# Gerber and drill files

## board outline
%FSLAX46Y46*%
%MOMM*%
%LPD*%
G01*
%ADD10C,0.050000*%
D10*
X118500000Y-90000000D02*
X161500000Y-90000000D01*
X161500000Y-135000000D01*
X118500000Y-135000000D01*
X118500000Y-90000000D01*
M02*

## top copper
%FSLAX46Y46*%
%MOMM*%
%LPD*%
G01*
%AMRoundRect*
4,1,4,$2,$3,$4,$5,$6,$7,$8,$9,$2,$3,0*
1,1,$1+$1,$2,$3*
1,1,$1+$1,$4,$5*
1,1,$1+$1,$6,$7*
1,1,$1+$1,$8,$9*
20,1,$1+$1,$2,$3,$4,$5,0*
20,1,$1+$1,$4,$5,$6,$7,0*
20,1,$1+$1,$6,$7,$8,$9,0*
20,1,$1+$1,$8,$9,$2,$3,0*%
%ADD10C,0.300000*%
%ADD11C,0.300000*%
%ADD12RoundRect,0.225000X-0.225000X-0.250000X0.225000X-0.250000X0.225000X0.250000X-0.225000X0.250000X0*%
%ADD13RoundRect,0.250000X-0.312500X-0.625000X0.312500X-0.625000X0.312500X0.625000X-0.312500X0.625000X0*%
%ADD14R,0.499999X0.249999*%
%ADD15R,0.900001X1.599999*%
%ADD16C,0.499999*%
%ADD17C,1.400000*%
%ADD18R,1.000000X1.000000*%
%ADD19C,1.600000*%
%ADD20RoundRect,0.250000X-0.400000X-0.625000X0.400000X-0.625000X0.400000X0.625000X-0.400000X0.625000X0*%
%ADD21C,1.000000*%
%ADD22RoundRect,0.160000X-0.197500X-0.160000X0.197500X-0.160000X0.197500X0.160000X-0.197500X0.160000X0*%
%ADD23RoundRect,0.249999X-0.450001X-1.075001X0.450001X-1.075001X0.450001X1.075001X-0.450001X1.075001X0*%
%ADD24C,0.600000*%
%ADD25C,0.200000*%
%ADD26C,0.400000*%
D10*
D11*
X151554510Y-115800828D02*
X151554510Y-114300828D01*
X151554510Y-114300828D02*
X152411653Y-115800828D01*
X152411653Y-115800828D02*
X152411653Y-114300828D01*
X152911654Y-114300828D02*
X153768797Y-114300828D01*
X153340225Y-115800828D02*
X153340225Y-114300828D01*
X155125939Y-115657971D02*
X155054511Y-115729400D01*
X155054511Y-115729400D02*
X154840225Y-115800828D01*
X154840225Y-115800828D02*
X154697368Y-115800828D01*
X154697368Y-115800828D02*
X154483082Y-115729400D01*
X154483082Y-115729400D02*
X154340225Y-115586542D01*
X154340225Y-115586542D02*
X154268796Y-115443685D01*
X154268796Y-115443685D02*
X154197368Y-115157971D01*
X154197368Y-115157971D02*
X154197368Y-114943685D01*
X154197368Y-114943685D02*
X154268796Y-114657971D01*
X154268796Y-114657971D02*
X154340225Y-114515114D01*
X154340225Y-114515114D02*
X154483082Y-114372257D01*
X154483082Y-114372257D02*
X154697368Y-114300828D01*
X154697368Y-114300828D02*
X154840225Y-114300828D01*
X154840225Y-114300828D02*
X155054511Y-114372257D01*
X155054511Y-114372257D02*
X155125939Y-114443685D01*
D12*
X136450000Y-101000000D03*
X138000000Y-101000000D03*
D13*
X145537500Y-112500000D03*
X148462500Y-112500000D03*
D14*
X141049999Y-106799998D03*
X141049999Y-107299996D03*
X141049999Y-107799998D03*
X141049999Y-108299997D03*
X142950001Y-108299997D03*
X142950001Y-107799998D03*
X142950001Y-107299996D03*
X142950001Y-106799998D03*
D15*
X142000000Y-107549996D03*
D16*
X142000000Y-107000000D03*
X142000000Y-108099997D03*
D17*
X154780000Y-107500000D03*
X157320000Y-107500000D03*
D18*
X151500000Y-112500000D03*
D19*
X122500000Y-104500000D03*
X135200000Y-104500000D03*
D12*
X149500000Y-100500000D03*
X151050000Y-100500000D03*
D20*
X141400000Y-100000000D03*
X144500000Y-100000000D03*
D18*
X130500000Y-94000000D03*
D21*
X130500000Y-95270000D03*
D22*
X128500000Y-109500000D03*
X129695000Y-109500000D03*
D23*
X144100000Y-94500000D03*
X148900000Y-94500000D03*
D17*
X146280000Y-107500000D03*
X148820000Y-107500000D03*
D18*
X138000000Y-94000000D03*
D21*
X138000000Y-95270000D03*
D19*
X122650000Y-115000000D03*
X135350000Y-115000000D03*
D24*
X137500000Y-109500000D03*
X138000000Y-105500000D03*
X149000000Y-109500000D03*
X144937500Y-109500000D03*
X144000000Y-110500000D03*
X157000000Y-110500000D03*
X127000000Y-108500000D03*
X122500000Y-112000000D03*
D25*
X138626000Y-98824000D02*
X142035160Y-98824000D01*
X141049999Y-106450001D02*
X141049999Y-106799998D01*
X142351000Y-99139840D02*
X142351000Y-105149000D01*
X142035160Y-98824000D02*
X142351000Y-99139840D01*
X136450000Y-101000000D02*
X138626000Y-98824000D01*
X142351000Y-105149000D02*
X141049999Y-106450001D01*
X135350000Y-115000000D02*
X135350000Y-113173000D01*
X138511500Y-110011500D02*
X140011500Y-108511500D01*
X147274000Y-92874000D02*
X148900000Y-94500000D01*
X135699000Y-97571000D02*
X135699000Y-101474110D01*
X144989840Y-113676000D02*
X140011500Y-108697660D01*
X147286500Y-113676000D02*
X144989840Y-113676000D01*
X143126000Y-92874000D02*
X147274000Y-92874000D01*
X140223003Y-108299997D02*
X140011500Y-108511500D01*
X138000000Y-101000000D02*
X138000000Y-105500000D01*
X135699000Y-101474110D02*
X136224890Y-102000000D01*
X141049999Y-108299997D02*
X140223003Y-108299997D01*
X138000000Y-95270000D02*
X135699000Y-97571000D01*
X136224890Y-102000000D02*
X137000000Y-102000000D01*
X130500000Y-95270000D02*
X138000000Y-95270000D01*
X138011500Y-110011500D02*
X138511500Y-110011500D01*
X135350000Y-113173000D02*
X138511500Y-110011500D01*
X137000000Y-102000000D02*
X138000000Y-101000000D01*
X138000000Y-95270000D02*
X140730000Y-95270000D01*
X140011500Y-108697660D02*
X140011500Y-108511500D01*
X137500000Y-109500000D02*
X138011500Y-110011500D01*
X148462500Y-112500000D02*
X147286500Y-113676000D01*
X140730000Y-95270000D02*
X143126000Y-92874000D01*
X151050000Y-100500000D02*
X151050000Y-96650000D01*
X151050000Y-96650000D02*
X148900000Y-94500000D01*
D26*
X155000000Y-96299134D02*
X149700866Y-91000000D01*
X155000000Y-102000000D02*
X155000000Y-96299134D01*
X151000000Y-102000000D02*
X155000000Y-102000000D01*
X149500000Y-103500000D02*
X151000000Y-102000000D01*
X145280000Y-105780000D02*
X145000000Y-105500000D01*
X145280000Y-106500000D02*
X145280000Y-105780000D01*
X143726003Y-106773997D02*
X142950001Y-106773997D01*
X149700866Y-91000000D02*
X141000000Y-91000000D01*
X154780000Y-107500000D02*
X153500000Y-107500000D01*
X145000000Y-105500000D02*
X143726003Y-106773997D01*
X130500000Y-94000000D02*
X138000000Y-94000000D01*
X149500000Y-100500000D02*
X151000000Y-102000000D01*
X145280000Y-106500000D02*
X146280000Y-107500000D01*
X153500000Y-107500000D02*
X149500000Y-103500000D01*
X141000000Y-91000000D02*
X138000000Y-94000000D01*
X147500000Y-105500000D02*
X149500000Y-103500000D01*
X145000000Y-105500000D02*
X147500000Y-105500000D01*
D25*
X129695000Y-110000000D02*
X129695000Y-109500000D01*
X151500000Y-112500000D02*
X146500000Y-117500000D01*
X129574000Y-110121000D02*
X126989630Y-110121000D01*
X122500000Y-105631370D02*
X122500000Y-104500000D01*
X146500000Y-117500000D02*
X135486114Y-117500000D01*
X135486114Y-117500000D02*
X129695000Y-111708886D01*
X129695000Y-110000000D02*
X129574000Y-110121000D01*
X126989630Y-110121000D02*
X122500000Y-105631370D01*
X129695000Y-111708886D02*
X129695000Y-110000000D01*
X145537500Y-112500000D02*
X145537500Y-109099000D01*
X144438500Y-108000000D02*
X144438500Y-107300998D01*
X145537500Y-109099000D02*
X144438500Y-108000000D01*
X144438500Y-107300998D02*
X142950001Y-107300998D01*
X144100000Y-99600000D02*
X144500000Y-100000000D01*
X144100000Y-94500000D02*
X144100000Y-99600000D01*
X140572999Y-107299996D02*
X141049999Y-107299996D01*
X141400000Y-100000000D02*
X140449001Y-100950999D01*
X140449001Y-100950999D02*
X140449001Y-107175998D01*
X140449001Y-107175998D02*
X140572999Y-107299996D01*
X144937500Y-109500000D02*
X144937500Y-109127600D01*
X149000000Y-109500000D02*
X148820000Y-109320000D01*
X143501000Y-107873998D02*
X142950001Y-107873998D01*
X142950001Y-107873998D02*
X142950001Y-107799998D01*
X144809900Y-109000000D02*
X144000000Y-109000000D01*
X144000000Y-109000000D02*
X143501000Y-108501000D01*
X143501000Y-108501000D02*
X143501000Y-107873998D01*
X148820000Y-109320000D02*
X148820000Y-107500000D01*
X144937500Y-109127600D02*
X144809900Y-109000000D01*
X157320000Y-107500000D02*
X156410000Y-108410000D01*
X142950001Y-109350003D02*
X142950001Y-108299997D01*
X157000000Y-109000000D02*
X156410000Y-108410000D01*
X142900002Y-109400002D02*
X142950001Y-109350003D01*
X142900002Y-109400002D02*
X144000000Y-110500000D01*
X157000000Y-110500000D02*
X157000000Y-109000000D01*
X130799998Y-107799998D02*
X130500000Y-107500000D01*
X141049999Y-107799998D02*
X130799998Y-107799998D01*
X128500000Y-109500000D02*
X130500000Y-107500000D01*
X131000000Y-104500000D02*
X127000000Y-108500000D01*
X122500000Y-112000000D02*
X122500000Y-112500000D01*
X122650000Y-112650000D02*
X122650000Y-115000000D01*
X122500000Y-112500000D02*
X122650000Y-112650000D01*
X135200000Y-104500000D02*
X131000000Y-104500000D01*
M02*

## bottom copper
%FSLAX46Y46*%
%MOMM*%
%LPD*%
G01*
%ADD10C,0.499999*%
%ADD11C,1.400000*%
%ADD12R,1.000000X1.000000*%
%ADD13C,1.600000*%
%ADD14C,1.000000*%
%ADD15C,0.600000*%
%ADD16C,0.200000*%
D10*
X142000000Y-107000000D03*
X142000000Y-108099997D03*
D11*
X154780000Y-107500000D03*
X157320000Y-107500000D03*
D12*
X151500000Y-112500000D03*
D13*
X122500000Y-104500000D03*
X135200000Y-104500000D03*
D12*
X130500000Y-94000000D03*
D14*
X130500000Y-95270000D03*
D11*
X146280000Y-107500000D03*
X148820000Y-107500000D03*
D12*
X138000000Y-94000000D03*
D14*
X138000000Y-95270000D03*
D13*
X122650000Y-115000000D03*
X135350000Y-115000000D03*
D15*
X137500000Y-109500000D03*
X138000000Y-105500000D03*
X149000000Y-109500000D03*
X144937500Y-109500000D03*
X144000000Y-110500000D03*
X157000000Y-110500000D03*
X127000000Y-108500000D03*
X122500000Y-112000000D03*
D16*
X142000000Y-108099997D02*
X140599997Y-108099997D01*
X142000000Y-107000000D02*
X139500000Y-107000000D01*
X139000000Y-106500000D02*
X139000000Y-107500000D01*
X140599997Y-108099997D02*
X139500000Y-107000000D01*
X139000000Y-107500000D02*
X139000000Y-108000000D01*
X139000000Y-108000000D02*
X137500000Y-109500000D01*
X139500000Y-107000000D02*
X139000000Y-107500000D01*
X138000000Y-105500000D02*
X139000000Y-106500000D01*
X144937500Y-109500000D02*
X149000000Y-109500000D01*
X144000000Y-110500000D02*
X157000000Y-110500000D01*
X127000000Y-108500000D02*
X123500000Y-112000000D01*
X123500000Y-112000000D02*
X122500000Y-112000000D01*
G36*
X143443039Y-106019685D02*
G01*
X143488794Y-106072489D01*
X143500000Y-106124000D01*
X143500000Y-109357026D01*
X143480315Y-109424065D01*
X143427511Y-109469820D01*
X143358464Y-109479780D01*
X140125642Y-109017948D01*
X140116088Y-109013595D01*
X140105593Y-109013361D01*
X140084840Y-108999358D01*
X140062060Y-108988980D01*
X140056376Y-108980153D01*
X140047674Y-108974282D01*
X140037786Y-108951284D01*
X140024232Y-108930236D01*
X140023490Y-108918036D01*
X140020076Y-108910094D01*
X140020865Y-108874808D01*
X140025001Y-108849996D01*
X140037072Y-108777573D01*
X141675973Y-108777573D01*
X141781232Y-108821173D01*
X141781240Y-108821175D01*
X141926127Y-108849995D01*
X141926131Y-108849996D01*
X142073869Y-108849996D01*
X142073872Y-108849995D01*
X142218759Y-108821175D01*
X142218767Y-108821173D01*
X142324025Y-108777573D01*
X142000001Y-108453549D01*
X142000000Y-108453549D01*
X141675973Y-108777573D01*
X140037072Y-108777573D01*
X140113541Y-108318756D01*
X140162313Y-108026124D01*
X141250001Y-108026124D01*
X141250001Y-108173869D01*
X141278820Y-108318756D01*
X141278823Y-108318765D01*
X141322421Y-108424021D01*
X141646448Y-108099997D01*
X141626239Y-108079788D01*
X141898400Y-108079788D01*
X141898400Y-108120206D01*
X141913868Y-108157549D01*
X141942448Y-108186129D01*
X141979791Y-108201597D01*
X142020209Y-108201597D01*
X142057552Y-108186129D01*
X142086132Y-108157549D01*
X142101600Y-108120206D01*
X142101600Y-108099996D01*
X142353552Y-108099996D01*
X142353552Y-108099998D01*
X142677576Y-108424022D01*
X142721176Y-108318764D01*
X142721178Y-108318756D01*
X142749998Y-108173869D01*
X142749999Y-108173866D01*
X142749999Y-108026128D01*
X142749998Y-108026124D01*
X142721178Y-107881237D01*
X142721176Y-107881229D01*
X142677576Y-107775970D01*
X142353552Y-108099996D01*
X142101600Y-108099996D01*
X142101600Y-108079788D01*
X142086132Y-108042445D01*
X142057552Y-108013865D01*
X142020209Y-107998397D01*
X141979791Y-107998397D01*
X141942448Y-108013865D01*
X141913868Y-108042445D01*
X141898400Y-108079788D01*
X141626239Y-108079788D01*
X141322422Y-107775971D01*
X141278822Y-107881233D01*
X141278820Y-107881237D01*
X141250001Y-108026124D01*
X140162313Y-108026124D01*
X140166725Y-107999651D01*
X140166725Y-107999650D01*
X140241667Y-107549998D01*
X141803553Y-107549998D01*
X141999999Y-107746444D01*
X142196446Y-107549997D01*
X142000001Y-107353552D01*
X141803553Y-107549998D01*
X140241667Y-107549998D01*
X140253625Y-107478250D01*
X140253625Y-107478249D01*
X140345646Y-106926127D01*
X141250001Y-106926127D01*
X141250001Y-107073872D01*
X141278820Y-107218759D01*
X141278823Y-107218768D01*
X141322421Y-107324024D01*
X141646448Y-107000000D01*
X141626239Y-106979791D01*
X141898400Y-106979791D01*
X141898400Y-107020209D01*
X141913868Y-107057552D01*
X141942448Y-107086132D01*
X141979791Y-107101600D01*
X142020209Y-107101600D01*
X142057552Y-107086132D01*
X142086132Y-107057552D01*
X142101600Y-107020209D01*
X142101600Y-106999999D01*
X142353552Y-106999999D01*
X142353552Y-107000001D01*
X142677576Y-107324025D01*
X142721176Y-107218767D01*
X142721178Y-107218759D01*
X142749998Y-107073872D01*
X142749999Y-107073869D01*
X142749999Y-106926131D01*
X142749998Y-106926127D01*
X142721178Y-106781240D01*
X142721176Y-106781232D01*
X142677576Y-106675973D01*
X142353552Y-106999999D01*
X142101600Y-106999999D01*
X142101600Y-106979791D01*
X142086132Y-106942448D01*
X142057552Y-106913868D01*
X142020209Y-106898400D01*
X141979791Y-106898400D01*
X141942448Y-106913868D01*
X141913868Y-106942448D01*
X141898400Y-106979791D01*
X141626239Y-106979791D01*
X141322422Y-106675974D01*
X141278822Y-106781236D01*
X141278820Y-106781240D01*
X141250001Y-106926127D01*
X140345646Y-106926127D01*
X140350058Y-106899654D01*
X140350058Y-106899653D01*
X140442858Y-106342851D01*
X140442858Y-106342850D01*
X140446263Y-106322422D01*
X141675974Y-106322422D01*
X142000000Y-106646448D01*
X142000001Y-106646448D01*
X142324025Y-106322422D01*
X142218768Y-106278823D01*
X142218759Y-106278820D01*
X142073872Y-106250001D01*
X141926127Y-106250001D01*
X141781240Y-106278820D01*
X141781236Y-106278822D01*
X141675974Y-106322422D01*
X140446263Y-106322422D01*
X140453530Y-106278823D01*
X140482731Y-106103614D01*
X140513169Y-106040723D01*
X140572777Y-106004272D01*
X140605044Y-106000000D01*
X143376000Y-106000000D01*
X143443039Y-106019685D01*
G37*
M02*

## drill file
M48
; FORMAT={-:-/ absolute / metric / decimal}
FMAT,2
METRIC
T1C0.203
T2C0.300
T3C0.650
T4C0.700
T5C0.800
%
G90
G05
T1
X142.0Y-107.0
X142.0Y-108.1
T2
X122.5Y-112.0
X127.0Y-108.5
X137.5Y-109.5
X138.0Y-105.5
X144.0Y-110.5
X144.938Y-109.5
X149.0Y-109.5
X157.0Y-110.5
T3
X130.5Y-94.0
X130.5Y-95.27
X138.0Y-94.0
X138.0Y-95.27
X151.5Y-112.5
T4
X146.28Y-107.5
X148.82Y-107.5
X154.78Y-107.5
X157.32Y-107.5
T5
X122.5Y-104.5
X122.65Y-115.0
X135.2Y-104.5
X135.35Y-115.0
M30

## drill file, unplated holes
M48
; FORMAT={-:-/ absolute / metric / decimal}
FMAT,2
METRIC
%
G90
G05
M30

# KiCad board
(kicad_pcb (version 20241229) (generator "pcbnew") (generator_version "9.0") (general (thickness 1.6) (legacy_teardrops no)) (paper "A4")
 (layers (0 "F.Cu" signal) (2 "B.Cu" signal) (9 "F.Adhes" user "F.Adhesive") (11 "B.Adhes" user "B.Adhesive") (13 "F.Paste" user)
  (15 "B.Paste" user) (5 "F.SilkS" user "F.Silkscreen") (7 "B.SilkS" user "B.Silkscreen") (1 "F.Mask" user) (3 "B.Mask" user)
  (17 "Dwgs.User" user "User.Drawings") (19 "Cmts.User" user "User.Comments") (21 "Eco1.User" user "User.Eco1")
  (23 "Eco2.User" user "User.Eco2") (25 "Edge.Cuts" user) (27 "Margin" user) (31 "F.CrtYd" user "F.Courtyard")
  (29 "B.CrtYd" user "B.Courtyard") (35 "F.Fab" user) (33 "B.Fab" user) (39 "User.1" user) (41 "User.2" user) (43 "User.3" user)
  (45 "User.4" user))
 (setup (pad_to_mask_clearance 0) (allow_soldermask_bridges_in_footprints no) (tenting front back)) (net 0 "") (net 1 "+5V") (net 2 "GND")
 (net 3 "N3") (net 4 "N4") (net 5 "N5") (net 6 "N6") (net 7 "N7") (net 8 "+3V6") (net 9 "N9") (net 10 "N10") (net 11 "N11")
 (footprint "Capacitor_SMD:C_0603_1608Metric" (layer "F.Cu") (at 137.225 101)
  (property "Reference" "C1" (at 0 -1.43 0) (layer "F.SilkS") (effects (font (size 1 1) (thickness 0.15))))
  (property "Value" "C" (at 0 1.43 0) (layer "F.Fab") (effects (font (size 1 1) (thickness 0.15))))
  (pad "1" smd roundrect (at -0.775 0) (size 0.9 0.95) (layers "F.Cu" "F.Mask" "F.Paste") (roundrect_rratio 0.25) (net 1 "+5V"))
  (pad "2" smd roundrect (at 0.775 0) (size 0.9 0.95) (layers "F.Cu" "F.Mask" "F.Paste") (roundrect_rratio 0.25) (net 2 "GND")))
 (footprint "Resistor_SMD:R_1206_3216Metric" (layer "F.Cu") (at 147 112.5)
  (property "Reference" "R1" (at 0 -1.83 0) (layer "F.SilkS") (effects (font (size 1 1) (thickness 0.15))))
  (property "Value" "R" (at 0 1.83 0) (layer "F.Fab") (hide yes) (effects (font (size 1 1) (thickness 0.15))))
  (pad "1" smd roundrect (at -1.4625 0) (size 1.125 1.75) (layers "F.Cu" "F.Mask" "F.Paste") (roundrect_rratio 0.222222) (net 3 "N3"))
  (pad "2" smd roundrect (at 1.4625 0) (size 1.125 1.75) (layers "F.Cu" "F.Mask" "F.Paste") (roundrect_rratio 0.222222) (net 2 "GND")))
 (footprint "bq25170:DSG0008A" (layer "F.Cu") (at 142 107.549996)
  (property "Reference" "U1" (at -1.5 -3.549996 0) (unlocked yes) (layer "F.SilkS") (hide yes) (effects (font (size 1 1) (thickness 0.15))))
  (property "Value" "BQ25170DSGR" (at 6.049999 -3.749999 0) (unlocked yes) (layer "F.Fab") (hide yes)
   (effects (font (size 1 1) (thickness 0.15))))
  (pad "1" smd rect (at -0.950001 -0.749998 90) (size 0.249999 0.499999) (layers "F.Cu" "F.Mask" "F.Paste") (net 1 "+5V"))
  (pad "2" smd rect (at -0.950001 -0.25 90) (size 0.249999 0.499999) (layers "F.Cu" "F.Mask" "F.Paste") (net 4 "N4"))
  (pad "3" smd rect (at -0.950001 0.250002 90) (size 0.249999 0.499999) (layers "F.Cu" "F.Mask" "F.Paste") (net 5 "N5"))
  (pad "4" smd rect (at -0.950001 0.750001 90) (size 0.249999 0.499999) (layers "F.Cu" "F.Mask" "F.Paste") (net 2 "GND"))
  (pad "5" smd rect (at 0.950001 0.750001 90) (size 0.249999 0.499999) (layers "F.Cu" "F.Mask" "F.Paste") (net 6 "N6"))
  (pad "6" smd rect (at 0.950001 0.250002 90) (size 0.249999 0.499999) (layers "F.Cu" "F.Mask" "F.Paste") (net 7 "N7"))
  (pad "7" smd rect (at 0.950001 -0.25 90) (size 0.249999 0.499999) (layers "F.Cu" "F.Mask" "F.Paste") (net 3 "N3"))
  (pad "8" smd rect (at 0.950001 -0.749998 90) (size 0.249999 0.499999) (layers "F.Cu" "F.Mask" "F.Paste") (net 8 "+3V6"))
  (pad "9" smd rect (at 0 0) (size 0.900001 1.599999) (layers "F.Cu" "F.Mask" "F.Paste") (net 2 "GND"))
  (pad "10" thru_hole circle (at 0 -0.549996) (size 0.499999 0.499999) (drill 0.2032) (layers "*.Cu" "*.Mask") (remove_unused_layers yes)
   (keep_end_layers yes) (zone_layer_connections) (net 2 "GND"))
  (pad "11" thru_hole circle (at 0 0.550001) (size 0.499999 0.499999) (drill 0.2032) (layers "*.Cu" "*.Mask") (remove_unused_layers yes)
   (keep_end_layers yes) (zone_layer_connections) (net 2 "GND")))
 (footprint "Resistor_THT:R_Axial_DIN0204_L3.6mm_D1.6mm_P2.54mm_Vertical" (layer "F.Cu") (at 154.78 107.5)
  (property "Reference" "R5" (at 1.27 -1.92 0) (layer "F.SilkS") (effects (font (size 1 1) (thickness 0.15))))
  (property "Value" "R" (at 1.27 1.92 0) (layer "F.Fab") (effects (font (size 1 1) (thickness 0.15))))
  (pad "1" thru_hole circle (at 0 0) (size 1.4 1.4) (drill 0.7) (layers "*.Cu" "*.Mask") (remove_unused_layers yes) (keep_end_layers yes)
   (zone_layer_connections) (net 8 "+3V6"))
  (pad "2" thru_hole circle (at 2.54 0) (size 1.4 1.4) (drill 0.7) (layers "*.Cu" "*.Mask") (remove_unused_layers yes) (keep_end_layers yes)
   (zone_layer_connections) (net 6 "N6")))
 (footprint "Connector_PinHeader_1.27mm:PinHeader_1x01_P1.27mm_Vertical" (layer "F.Cu") (at 151.5 112.5)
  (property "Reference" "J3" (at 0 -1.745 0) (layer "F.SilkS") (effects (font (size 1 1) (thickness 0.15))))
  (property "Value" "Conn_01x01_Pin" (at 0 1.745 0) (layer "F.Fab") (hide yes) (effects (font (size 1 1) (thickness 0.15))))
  (pad "1" thru_hole rect (at 0 0) (size 1 1) (drill 0.65) (layers "*.Cu" "*.Mask") (remove_unused_layers yes) (keep_end_layers yes)
   (zone_layer_connections) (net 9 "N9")))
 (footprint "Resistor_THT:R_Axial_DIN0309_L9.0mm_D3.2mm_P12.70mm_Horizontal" (layer "F.Cu") (at 122.5 104.5)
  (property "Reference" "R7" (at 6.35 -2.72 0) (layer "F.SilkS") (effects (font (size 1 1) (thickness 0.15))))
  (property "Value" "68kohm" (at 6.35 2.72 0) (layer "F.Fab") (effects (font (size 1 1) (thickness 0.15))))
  (pad "1" thru_hole circle (at 0 0) (size 1.6 1.6) (drill 0.8) (layers "*.Cu" "*.Mask") (remove_unused_layers yes) (keep_end_layers yes)
   (zone_layer_connections) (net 9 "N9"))
  (pad "2" thru_hole circle (at 12.7 0) (size 1.6 1.6) (drill 0.8) (layers "*.Cu" "*.Mask") (remove_unused_layers yes) (keep_end_layers yes)
   (zone_layer_connections) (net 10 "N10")))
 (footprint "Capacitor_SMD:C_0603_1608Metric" (layer "F.Cu") (at 150.275 100.5)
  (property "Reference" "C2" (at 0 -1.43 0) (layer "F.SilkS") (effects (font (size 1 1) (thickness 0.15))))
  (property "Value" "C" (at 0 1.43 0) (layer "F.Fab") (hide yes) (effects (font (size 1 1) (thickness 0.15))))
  (pad "1" smd roundrect (at -0.775 0) (size 0.9 0.95) (layers "F.Cu" "F.Mask" "F.Paste") (roundrect_rratio 0.25) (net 8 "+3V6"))
  (pad "2" smd roundrect (at 0.775 0) (size 0.9 0.95) (layers "F.Cu" "F.Mask" "F.Paste") (roundrect_rratio 0.25) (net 2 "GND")))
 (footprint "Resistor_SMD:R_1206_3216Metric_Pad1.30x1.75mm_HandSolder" (layer "F.Cu") (at 142.95 100)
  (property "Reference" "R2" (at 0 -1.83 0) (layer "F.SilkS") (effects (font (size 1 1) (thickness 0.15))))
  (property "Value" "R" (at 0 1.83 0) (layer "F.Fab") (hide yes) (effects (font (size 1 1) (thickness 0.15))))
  (pad "1" smd roundrect (at -1.55 0) (size 1.3 1.75) (layers "F.Cu" "F.Mask" "F.Paste") (roundrect_rratio 0.192308) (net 4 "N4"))
  (pad "2" smd roundrect (at 1.55 0) (size 1.3 1.75) (layers "F.Cu" "F.Mask" "F.Paste") (roundrect_rratio 0.192308) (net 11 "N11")))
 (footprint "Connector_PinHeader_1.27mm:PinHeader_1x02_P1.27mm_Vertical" (layer "F.Cu") (at 130.5 94)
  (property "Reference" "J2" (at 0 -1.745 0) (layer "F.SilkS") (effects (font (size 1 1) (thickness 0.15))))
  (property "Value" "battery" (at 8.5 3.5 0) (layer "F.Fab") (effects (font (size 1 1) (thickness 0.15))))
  (pad "1" thru_hole rect (at 0 0) (size 1 1) (drill 0.65) (layers "*.Cu" "*.Mask") (remove_unused_layers yes) (keep_end_layers yes)
   (zone_layer_connections) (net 8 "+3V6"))
  (pad "2" thru_hole circle (at 0 1.27) (size 1 1) (drill 0.65) (layers "*.Cu" "*.Mask") (remove_unused_layers yes) (keep_end_layers yes)
   (zone_layer_connections) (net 2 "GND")))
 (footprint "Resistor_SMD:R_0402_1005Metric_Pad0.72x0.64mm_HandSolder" (layer "F.Cu") (at 129.0975 109.5)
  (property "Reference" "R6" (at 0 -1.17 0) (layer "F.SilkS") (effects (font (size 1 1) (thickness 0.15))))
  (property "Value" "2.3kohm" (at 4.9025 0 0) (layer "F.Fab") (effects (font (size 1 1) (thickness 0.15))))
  (pad "1" smd roundrect (at -0.5975 0) (size 0.715 0.64) (layers "F.Cu" "F.Mask" "F.Paste") (roundrect_rratio 0.25) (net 5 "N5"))
  (pad "2" smd roundrect (at 0.5975 0) (size 0.715 0.64) (layers "F.Cu" "F.Mask" "F.Paste") (roundrect_rratio 0.25) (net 9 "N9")))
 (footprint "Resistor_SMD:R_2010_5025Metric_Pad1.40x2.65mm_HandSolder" (layer "F.Cu") (at 146.5 94.5)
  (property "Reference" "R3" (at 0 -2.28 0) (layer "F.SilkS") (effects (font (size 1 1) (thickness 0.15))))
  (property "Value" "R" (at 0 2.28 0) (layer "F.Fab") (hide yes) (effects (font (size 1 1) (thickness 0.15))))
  (pad "1" smd roundrect (at -2.4 0) (size 1.4 2.65) (layers "F.Cu" "F.Mask" "F.Paste") (roundrect_rratio 0.178571) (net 11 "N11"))
  (pad "2" smd roundrect (at 2.4 0) (size 1.4 2.65) (layers "F.Cu" "F.Mask" "F.Paste") (roundrect_rratio 0.178571) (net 2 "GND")))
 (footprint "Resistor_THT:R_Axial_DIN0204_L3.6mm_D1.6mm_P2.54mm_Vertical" (layer "F.Cu") (at 146.28 107.5)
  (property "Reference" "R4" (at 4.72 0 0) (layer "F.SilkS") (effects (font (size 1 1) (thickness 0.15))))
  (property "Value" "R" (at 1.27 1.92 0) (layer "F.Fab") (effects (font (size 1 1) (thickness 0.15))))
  (pad "1" thru_hole circle (at 0 0) (size 1.4 1.4) (drill 0.7) (layers "*.Cu" "*.Mask") (remove_unused_layers yes) (keep_end_layers yes)
   (zone_layer_connections) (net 8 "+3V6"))
  (pad "2" thru_hole circle (at 2.54 0) (size 1.4 1.4) (drill 0.7) (layers "*.Cu" "*.Mask") (remove_unused_layers yes) (keep_end_layers yes)
   (zone_layer_connections) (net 7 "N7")))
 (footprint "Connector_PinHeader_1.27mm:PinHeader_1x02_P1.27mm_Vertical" (layer "F.Cu") (at 138 94)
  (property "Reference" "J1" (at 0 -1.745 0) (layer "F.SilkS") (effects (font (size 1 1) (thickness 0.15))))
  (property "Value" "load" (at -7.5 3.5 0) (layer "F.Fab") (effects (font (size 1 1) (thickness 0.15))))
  (pad "1" thru_hole rect (at 0 0) (size 1 1) (drill 0.65) (layers "*.Cu" "*.Mask") (remove_unused_layers yes) (keep_end_layers yes)
   (zone_layer_connections) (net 8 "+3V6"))
  (pad "2" thru_hole circle (at 0 1.27) (size 1 1) (drill 0.65) (layers "*.Cu" "*.Mask") (remove_unused_layers yes) (keep_end_layers yes)
   (zone_layer_connections) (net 2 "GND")))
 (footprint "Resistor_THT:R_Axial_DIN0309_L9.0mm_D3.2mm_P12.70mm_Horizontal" (layer "F.Cu") (at 122.65 115)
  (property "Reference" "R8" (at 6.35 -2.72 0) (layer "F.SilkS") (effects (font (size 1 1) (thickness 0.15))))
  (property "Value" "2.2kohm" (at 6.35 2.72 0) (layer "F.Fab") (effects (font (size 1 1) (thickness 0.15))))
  (pad "1" thru_hole circle (at 0 0) (size 1.6 1.6) (drill 0.8) (layers "*.Cu" "*.Mask") (remove_unused_layers yes) (keep_end_layers yes)
   (zone_layer_connections) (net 10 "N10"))
  (pad "2" thru_hole circle (at 12.7 0) (size 1.6 1.6) (drill 0.8) (layers "*.Cu" "*.Mask") (remove_unused_layers yes) (keep_end_layers yes)
   (zone_layer_connections) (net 2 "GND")))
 (gr_rect (start 118.5 90) (end 161.5 135) (stroke (width 0.05) (type default)) (fill no) (layer "Edge.Cuts"))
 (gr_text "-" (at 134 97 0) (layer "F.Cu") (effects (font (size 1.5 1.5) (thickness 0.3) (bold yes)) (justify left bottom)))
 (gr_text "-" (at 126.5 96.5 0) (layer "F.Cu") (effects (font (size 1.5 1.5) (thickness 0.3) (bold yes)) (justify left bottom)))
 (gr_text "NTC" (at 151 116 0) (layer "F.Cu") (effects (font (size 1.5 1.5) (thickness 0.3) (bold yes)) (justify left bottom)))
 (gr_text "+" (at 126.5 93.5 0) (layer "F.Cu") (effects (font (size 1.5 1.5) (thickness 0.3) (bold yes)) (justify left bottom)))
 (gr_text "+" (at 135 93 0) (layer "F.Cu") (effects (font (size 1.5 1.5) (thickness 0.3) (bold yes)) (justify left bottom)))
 (segment (start 138.626 98.824) (end 142.03516 98.824) (width 0.2) (layer "F.Cu") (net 1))
 (segment (start 141.049999 106.450001) (end 141.049999 106.799998) (width 0.2) (layer "F.Cu") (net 1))
 (segment (start 142.351 99.13984) (end 142.351 105.149) (width 0.2) (layer "F.Cu") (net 1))
 (segment (start 142.03516 98.824) (end 142.351 99.13984) (width 0.2) (layer "F.Cu") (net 1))
 (segment (start 136.45 101) (end 138.626 98.824) (width 0.2) (layer "F.Cu") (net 1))
 (segment (start 142.351 105.149) (end 141.049999 106.450001) (width 0.2) (layer "F.Cu") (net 1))
 (segment (start 135.35 115) (end 135.35 113.173) (width 0.2) (layer "F.Cu") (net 2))
 (segment (start 138.5115 110.0115) (end 140.0115 108.5115) (width 0.2) (layer "F.Cu") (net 2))
 (segment (start 147.274 92.874) (end 148.9 94.5) (width 0.2) (layer "F.Cu") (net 2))
 (segment (start 135.699 97.571) (end 135.699 101.47411) (width 0.2) (layer "F.Cu") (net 2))
 (segment (start 144.98984 113.676) (end 140.0115 108.69766) (width 0.2) (layer "F.Cu") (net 2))
 (segment (start 147.2865 113.676) (end 144.98984 113.676) (width 0.2) (layer "F.Cu") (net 2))
 (segment (start 143.126 92.874) (end 147.274 92.874) (width 0.2) (layer "F.Cu") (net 2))
 (segment (start 140.223003 108.299997) (end 140.0115 108.5115) (width 0.2) (layer "F.Cu") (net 2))
 (segment (start 138 101) (end 138 105.5) (width 0.2) (layer "F.Cu") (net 2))
 (segment (start 135.699 101.47411) (end 136.22489 102) (width 0.2) (layer "F.Cu") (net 2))
 (segment (start 141.049999 108.299997) (end 140.223003 108.299997) (width 0.2) (layer "F.Cu") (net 2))
 (segment (start 138 95.27) (end 135.699 97.571) (width 0.2) (layer "F.Cu") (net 2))
 (segment (start 136.22489 102) (end 137 102) (width 0.2) (layer "F.Cu") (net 2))
 (segment (start 130.5 95.27) (end 138 95.27) (width 0.2) (layer "F.Cu") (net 2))
 (segment (start 138.0115 110.0115) (end 138.5115 110.0115) (width 0.2) (layer "F.Cu") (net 2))
 (segment (start 135.35 113.173) (end 138.5115 110.0115) (width 0.2) (layer "F.Cu") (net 2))
 (segment (start 137 102) (end 138 101) (width 0.2) (layer "F.Cu") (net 2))
 (segment (start 138 95.27) (end 140.73 95.27) (width 0.2) (layer "F.Cu") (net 2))
 (segment (start 140.0115 108.69766) (end 140.0115 108.5115) (width 0.2) (layer "F.Cu") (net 2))
 (segment (start 137.5 109.5) (end 138.0115 110.0115) (width 0.2) (layer "F.Cu") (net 2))
 (segment (start 148.4625 112.5) (end 147.2865 113.676) (width 0.2) (layer "F.Cu") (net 2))
 (segment (start 140.73 95.27) (end 143.126 92.874) (width 0.2) (layer "F.Cu") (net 2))
 (segment (start 151.05 100.5) (end 151.05 96.65) (width 0.2) (layer "F.Cu") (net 2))
 (segment (start 151.05 96.65) (end 148.9 94.5) (width 0.2) (layer "F.Cu") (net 2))
 (via (at 137.5 109.5) (size 0.6) (drill 0.3) (layers "F.Cu" "B.Cu") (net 2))
 (via (at 138 105.5) (size 0.6) (drill 0.3) (layers "F.Cu" "B.Cu") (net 2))
 (segment (start 142 108.099997) (end 140.599997 108.099997) (width 0.2) (layer "B.Cu") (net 2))
 (segment (start 142 107) (end 139.5 107) (width 0.2) (layer "B.Cu") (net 2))
 (segment (start 139 106.5) (end 139 107.5) (width 0.2) (layer "B.Cu") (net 2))
 (segment (start 140.599997 108.099997) (end 139.5 107) (width 0.2) (layer "B.Cu") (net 2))
 (segment (start 139 107.5) (end 139 108) (width 0.2) (layer "B.Cu") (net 2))
 (segment (start 139 108) (end 137.5 109.5) (width 0.2) (layer "B.Cu") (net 2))
 (segment (start 139.5 107) (end 139 107.5) (width 0.2) (layer "B.Cu") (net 2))
 (segment (start 138 105.5) (end 139 106.5) (width 0.2) (layer "B.Cu") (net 2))
 (segment (start 155 96.299134) (end 149.700866 91) (width 0.4) (layer "F.Cu") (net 8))
 (segment (start 155 102) (end 155 96.299134) (width 0.4) (layer "F.Cu") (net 8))
 (segment (start 151 102) (end 155 102) (width 0.4) (layer "F.Cu") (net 8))
 (segment (start 149.5 103.5) (end 151 102) (width 0.4) (layer "F.Cu") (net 8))
 (segment (start 145.28 105.78) (end 145 105.5) (width 0.4) (layer "F.Cu") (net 8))
 (segment (start 145.28 106.5) (end 145.28 105.78) (width 0.4) (layer "F.Cu") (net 8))
 (segment (start 143.726003 106.773997) (end 142.950001 106.773997) (width 0.4) (layer "F.Cu") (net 8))
 (segment (start 149.700866 91) (end 141 91) (width 0.4) (layer "F.Cu") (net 8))
 (segment (start 154.78 107.5) (end 153.5 107.5) (width 0.4) (layer "F.Cu") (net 8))
 (segment (start 145 105.5) (end 143.726003 106.773997) (width 0.4) (layer "F.Cu") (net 8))
 (segment (start 130.5 94) (end 138 94) (width 0.4) (layer "F.Cu") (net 8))
 (segment (start 149.5 100.5) (end 151 102) (width 0.4) (layer "F.Cu") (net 8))
 (segment (start 145.28 106.5) (end 146.28 107.5) (width 0.4) (layer "F.Cu") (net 8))
 (segment (start 153.5 107.5) (end 149.5 103.5) (width 0.4) (layer "F.Cu") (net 8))
 (segment (start 141 91) (end 138 94) (width 0.4) (layer "F.Cu") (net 8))
 (segment (start 147.5 105.5) (end 149.5 103.5) (width 0.4) (layer "F.Cu") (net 8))
 (segment (start 145 105.5) (end 147.5 105.5) (width 0.4) (layer "F.Cu") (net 8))
 (segment (start 129.695 110) (end 129.695 109.5) (width 0.2) (layer "F.Cu") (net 9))
 (segment (start 151.5 112.5) (end 146.5 117.5) (width 0.2) (layer "F.Cu") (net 9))
 (segment (start 129.574 110.121) (end 126.98963 110.121) (width 0.2) (layer "F.Cu") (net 9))
 (segment (start 122.5 105.63137) (end 122.5 104.5) (width 0.2) (layer "F.Cu") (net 9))
 (segment (start 146.5 117.5) (end 135.486114 117.5) (width 0.2) (layer "F.Cu") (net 9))
 (segment (start 135.486114 117.5) (end 129.695 111.708886) (width 0.2) (layer "F.Cu") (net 9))
 (segment (start 129.695 110) (end 129.574 110.121) (width 0.2) (layer "F.Cu") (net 9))
 (segment (start 126.98963 110.121) (end 122.5 105.63137) (width 0.2) (layer "F.Cu") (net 9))
 (segment (start 129.695 111.708886) (end 129.695 110) (width 0.2) (layer "F.Cu") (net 9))
 (segment (start 145.5375 112.5) (end 145.5375 109.099) (width 0.2) (layer "F.Cu") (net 3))
 (segment (start 144.4385 108) (end 144.4385 107.300998) (width 0.2) (layer "F.Cu") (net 3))
 (segment (start 145.5375 109.099) (end 144.4385 108) (width 0.2) (layer "F.Cu") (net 3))
 (segment (start 144.4385 107.300998) (end 142.950001 107.300998) (width 0.2) (layer "F.Cu") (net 3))
 (segment (start 144.1 99.6) (end 144.5 100) (width 0.2) (layer "F.Cu") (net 11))
 (segment (start 144.1 94.5) (end 144.1 99.6) (width 0.2) (layer "F.Cu") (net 11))
 (segment (start 140.572999 107.299996) (end 141.049999 107.299996) (width 0.2) (layer "F.Cu") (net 4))
 (segment (start 141.4 100) (end 140.449001 100.950999) (width 0.2) (layer "F.Cu") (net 4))
 (segment (start 140.449001 100.950999) (end 140.449001 107.175998) (width 0.2) (layer "F.Cu") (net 4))
 (segment (start 140.449001 107.175998) (end 140.572999 107.299996) (width 0.2) (layer "F.Cu") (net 4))
 (segment (start 144.9375 109.5) (end 144.9375 109.1276) (width 0.2) (layer "F.Cu") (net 7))
 (segment (start 149 109.5) (end 148.82 109.32) (width 0.2) (layer "F.Cu") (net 7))
 (segment (start 143.501 107.873998) (end 142.950001 107.873998) (width 0.2) (layer "F.Cu") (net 7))
 (segment (start 142.950001 107.873998) (end 142.950001 107.799998) (width 0.2) (layer "F.Cu") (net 7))
 (segment (start 144.8099 109) (end 144 109) (width 0.2) (layer "F.Cu") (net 7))
 (segment (start 144 109) (end 143.501 108.501) (width 0.2) (layer "F.Cu") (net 7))
 (segment (start 143.501 108.501) (end 143.501 107.873998) (width 0.2) (layer "F.Cu") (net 7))
 (segment (start 148.82 109.32) (end 148.82 107.5) (width 0.2) (layer "F.Cu") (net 7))
 (segment (start 144.9375 109.1276) (end 144.8099 109) (width 0.2) (layer "F.Cu") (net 7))
 (via (at 149 109.5) (size 0.6) (drill 0.3) (layers "F.Cu" "B.Cu") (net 7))
 (via (at 144.9375 109.5) (size 0.6) (drill 0.3) (layers "F.Cu" "B.Cu") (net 7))
 (segment (start 144.9375 109.5) (end 149 109.5) (width 0.2) (layer "B.Cu") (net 7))
 (segment (start 157.32 107.5) (end 156.41 108.41) (width 0.2) (layer "F.Cu") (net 6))
 (segment (start 142.950001 109.350003) (end 142.950001 108.299997) (width 0.2) (layer "F.Cu") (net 6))
 (segment (start 157 109) (end 156.41 108.41) (width 0.2) (layer "F.Cu") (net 6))
 (segment (start 142.900002 109.400002) (end 142.950001 109.350003) (width 0.2) (layer "F.Cu") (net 6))
 (segment (start 142.900002 109.400002) (end 144 110.5) (width 0.2) (layer "F.Cu") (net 6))
 (segment (start 157 110.5) (end 157 109) (width 0.2) (layer "F.Cu") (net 6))
 (via (at 144 110.5) (size 0.6) (drill 0.3) (layers "F.Cu" "B.Cu") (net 6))
 (via (at 157 110.5) (size 0.6) (drill 0.3) (layers "F.Cu" "B.Cu") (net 6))
 (segment (start 144 110.5) (end 157 110.5) (width 0.2) (layer "B.Cu") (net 6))
 (segment (start 130.799998 107.799998) (end 130.5 107.5) (width 0.2) (layer "F.Cu") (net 5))
 (segment (start 141.049999 107.799998) (end 130.799998 107.799998) (width 0.2) (layer "F.Cu") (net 5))
 (segment (start 128.5 109.5) (end 130.5 107.5) (width 0.2) (layer "F.Cu") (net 5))
 (segment (start 131 104.5) (end 127 108.5) (width 0.2) (layer "F.Cu") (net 10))
 (segment (start 122.5 112) (end 122.5 112.5) (width 0.2) (layer "F.Cu") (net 10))
 (segment (start 122.65 112.65) (end 122.65 115) (width 0.2) (layer "F.Cu") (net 10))
 (segment (start 122.5 112.5) (end 122.65 112.65) (width 0.2) (layer "F.Cu") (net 10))
 (segment (start 135.2 104.5) (end 131 104.5) (width 0.2) (layer "F.Cu") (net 10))
 (via (at 127 108.5) (size 0.6) (drill 0.3) (layers "F.Cu" "B.Cu") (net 10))
 (via (at 122.5 112) (size 0.6) (drill 0.3) (layers "F.Cu" "B.Cu") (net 10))
 (segment (start 127 108.5) (end 123.5 112) (width 0.2) (layer "B.Cu") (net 10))
 (segment (start 123.5 112) (end 122.5 112) (width 0.2) (layer "B.Cu") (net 10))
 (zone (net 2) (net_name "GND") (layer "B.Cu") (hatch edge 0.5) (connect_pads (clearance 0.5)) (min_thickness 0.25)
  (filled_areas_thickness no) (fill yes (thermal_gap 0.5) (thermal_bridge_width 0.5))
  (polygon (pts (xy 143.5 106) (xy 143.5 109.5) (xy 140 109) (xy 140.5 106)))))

